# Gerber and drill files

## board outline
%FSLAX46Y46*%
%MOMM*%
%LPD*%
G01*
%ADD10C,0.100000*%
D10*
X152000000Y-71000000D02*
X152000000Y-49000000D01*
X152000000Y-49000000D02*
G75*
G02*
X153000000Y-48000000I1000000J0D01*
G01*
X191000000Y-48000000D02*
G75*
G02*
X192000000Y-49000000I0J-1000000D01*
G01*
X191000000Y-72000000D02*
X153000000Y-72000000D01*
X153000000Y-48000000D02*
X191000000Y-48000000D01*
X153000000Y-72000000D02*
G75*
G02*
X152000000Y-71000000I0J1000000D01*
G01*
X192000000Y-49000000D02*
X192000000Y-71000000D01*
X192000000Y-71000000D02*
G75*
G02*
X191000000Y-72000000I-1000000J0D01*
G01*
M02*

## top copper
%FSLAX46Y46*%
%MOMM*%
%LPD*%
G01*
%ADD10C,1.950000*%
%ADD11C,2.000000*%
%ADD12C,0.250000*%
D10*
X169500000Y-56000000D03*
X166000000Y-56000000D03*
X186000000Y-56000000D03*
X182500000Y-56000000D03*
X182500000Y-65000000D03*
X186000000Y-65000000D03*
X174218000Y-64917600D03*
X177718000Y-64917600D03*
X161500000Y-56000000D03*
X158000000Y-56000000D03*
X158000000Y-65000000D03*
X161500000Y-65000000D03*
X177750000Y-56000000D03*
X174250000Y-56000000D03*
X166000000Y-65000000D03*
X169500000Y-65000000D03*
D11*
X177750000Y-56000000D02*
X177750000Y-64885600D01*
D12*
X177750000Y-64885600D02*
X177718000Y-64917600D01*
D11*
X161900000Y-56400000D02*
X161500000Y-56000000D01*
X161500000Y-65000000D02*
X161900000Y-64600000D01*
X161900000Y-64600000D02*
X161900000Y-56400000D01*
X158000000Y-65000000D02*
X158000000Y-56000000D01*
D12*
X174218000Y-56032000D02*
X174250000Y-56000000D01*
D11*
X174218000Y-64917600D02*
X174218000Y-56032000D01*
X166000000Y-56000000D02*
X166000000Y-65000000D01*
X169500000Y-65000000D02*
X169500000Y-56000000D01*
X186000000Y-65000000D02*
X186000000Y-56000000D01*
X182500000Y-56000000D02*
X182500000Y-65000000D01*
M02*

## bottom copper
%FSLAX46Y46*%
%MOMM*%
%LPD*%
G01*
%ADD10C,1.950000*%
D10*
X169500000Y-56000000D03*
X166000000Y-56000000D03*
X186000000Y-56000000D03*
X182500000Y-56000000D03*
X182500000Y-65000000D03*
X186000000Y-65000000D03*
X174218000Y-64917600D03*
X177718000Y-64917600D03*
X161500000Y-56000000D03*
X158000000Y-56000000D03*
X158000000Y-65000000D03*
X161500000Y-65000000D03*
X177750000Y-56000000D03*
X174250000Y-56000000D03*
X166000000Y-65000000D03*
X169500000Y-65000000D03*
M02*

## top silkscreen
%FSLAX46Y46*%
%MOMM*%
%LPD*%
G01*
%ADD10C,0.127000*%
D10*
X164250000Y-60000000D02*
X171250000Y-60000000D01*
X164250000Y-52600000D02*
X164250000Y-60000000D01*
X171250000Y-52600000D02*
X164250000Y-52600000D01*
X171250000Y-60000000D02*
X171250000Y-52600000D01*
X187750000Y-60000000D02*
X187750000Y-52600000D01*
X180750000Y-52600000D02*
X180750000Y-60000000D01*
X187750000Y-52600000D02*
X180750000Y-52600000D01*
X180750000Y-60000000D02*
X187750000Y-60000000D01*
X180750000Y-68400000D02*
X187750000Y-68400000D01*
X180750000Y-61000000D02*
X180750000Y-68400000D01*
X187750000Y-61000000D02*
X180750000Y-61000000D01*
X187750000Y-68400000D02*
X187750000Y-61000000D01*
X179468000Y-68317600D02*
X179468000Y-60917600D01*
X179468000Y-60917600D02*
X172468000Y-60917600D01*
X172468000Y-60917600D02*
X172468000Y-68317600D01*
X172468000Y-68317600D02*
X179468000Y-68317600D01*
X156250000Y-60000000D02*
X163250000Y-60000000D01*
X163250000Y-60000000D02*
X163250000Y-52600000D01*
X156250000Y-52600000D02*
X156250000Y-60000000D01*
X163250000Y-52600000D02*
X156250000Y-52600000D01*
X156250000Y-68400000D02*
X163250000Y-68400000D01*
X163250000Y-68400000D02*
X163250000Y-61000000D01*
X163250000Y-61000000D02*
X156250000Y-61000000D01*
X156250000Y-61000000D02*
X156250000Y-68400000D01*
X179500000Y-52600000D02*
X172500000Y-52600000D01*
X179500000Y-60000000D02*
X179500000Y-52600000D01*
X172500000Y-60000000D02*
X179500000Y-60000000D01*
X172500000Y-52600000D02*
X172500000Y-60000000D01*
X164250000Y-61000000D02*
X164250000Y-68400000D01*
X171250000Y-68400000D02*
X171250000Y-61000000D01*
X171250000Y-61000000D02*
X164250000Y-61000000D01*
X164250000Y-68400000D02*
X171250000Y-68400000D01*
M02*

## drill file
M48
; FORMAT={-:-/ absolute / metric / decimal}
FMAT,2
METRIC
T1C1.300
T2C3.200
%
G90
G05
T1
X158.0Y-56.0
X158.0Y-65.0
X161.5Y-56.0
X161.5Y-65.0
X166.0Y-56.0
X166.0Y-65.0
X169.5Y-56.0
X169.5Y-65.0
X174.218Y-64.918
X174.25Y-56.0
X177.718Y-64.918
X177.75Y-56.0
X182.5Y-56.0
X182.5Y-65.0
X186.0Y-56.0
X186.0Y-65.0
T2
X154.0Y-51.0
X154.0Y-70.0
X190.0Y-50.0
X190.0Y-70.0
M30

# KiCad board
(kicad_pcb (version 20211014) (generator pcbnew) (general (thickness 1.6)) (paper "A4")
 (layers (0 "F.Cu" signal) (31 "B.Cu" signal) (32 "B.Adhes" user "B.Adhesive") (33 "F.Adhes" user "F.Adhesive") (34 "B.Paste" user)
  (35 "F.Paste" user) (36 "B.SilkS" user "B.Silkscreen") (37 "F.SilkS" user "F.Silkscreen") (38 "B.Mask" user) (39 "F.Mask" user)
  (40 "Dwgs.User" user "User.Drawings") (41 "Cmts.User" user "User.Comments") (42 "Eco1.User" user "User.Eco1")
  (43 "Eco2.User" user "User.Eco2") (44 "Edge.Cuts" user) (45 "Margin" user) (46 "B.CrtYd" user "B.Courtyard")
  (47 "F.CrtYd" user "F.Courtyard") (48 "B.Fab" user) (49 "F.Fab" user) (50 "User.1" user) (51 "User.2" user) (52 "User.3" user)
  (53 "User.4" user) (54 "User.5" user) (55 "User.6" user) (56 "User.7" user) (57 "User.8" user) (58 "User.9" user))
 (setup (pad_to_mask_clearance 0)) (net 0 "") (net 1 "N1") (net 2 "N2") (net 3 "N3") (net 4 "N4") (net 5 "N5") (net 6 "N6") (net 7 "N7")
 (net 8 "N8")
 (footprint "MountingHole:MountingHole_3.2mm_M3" (layer "F.Cu") (at 154 51)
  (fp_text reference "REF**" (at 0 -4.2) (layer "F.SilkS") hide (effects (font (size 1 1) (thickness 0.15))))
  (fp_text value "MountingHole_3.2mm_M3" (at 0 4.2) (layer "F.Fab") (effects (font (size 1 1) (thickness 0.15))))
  (pad "" np_thru_hole circle (at 0 0) (size 3.2 3.2) (drill 3.2) (layers *.Cu *.Mask)))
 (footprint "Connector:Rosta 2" (layer "F.Cu") (at 167.75 56 180)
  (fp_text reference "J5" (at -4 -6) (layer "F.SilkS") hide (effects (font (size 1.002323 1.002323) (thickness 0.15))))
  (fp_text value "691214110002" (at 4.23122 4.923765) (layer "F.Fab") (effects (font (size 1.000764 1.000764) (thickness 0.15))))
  (fp_line (start 3.5 -4) (end -3.5 -4) (layer "F.SilkS") (width 0.127))
  (fp_line (start 3.5 3.4) (end 3.5 -4) (layer "F.SilkS") (width 0.127))
  (fp_line (start -3.5 3.4) (end 3.5 3.4) (layer "F.SilkS") (width 0.127))
  (fp_line (start -3.5 -4) (end -3.5 3.4) (layer "F.SilkS") (width 0.127))
  (pad "1" thru_hole circle (at -1.75 0 180) (size 1.95 1.95) (drill 1.3) (layers *.Cu *.Mask) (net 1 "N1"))
  (pad "2" thru_hole circle (at 1.75 0 180) (size 1.95 1.95) (drill 1.3) (layers *.Cu *.Mask) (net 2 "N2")))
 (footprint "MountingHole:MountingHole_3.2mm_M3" (layer "F.Cu") (at 190 50)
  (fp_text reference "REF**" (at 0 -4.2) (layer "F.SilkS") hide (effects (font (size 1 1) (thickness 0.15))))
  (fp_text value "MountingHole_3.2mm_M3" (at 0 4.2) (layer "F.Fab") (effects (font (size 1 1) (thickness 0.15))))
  (pad "" np_thru_hole circle (at 0 0) (size 3.2 3.2) (drill 3.2) (layers *.Cu *.Mask)))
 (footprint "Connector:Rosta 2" (layer "F.Cu") (at 184.25 56 180)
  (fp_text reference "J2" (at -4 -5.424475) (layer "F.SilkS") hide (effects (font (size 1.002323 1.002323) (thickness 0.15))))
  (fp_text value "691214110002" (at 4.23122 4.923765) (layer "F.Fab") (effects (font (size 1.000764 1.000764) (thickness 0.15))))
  (fp_line (start -3.5 -4) (end -3.5 3.4) (layer "F.SilkS") (width 0.127))
  (fp_line (start 3.5 3.4) (end 3.5 -4) (layer "F.SilkS") (width 0.127))
  (fp_line (start -3.5 3.4) (end 3.5 3.4) (layer "F.SilkS") (width 0.127))
  (fp_line (start 3.5 -4) (end -3.5 -4) (layer "F.SilkS") (width 0.127))
  (pad "1" thru_hole circle (at -1.75 0 180) (size 1.95 1.95) (drill 1.3) (layers *.Cu *.Mask) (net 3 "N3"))
  (pad "2" thru_hole circle (at 1.75 0 180) (size 1.95 1.95) (drill 1.3) (layers *.Cu *.Mask) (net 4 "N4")))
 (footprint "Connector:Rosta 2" (layer "F.Cu") (at 184.25 65)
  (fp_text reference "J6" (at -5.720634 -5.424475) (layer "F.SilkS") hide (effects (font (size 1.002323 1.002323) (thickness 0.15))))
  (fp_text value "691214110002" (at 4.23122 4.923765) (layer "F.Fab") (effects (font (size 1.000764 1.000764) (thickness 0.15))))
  (fp_line (start -3.5 3.4) (end 3.5 3.4) (layer "F.SilkS") (width 0.127))
  (fp_line (start -3.5 -4) (end -3.5 3.4) (layer "F.SilkS") (width 0.127))
  (fp_line (start 3.5 -4) (end -3.5 -4) (layer "F.SilkS") (width 0.127))
  (fp_line (start 3.5 3.4) (end 3.5 -4) (layer "F.SilkS") (width 0.127))
  (pad "1" thru_hole circle (at -1.75 0) (size 1.95 1.95) (drill 1.3) (layers *.Cu *.Mask) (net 4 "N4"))
  (pad "2" thru_hole circle (at 1.75 0) (size 1.95 1.95) (drill 1.3) (layers *.Cu *.Mask) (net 3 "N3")))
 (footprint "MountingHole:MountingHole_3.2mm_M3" (layer "F.Cu") (at 154 70)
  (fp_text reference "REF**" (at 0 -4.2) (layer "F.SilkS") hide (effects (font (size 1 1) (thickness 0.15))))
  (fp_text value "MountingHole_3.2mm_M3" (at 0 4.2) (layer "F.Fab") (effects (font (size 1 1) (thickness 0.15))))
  (pad "" np_thru_hole circle (at 0 0) (size 3.2 3.2) (drill 3.2) (layers *.Cu *.Mask)))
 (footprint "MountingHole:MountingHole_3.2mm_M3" (layer "F.Cu") (at 190 70)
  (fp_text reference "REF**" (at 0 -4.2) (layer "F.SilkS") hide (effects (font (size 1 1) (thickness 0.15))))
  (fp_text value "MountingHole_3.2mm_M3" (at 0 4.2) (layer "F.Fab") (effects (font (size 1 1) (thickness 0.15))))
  (pad "" np_thru_hole circle (at 0 0) (size 3.2 3.2) (drill 3.2) (layers *.Cu *.Mask)))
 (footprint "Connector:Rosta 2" (layer "F.Cu") (at 175.968 64.9176)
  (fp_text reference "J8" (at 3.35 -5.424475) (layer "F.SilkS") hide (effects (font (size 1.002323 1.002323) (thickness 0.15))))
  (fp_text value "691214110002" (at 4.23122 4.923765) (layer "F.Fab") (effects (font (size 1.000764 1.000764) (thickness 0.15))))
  (fp_line (start 3.5 3.4) (end 3.5 -4) (layer "F.SilkS") (width 0.127))
  (fp_line (start 3.5 -4) (end -3.5 -4) (layer "F.SilkS") (width 0.127))
  (fp_line (start -3.5 -4) (end -3.5 3.4) (layer "F.SilkS") (width 0.127))
  (fp_line (start -3.5 3.4) (end 3.5 3.4) (layer "F.SilkS") (width 0.127))
  (pad "1" thru_hole circle (at -1.75 0) (size 1.95 1.95) (drill 1.3) (layers *.Cu *.Mask) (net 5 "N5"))
  (pad "2" thru_hole circle (at 1.75 0) (size 1.95 1.95) (drill 1.3) (layers *.Cu *.Mask) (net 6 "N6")))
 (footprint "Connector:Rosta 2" (layer "F.Cu") (at 159.75 56 180)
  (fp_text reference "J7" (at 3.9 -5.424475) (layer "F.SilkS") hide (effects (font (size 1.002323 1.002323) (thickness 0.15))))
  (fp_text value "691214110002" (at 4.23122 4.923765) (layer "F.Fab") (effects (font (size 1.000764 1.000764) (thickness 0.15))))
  (fp_line (start 3.5 -4) (end -3.5 -4) (layer "F.SilkS") (width 0.127))
  (fp_line (start -3.5 -4) (end -3.5 3.4) (layer "F.SilkS") (width 0.127))
  (fp_line (start 3.5 3.4) (end 3.5 -4) (layer "F.SilkS") (width 0.127))
  (fp_line (start -3.5 3.4) (end 3.5 3.4) (layer "F.SilkS") (width 0.127))
  (pad "1" thru_hole circle (at -1.75 0 180) (size 1.95 1.95) (drill 1.3) (layers *.Cu *.Mask) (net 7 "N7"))
  (pad "2" thru_hole circle (at 1.75 0 180) (size 1.95 1.95) (drill 1.3) (layers *.Cu *.Mask) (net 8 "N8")))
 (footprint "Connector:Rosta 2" (layer "F.Cu") (at 159.75 65)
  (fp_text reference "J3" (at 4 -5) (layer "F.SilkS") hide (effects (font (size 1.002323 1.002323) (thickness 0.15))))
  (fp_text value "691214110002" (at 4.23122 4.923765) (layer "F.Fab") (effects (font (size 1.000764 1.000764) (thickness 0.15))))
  (fp_line (start -3.5 3.4) (end 3.5 3.4) (layer "F.SilkS") (width 0.127))
  (fp_line (start 3.5 3.4) (end 3.5 -4) (layer "F.SilkS") (width 0.127))
  (fp_line (start 3.5 -4) (end -3.5 -4) (layer "F.SilkS") (width 0.127))
  (fp_line (start -3.5 -4) (end -3.5 3.4) (layer "F.SilkS") (width 0.127))
  (pad "1" thru_hole circle (at -1.75 0) (size 1.95 1.95) (drill 1.3) (layers *.Cu *.Mask) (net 8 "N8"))
  (pad "2" thru_hole circle (at 1.75 0) (size 1.95 1.95) (drill 1.3) (layers *.Cu *.Mask) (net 7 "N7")))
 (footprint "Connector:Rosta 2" (layer "F.Cu") (at 176 56 180)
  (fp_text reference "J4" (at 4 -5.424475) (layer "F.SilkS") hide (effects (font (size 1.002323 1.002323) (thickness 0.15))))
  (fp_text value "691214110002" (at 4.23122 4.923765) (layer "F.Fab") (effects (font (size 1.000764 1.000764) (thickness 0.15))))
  (fp_line (start -3.5 3.4) (end 3.5 3.4) (layer "F.SilkS") (width 0.127))
  (fp_line (start -3.5 -4) (end -3.5 3.4) (layer "F.SilkS") (width 0.127))
  (fp_line (start 3.5 -4) (end -3.5 -4) (layer "F.SilkS") (width 0.127))
  (fp_line (start 3.5 3.4) (end 3.5 -4) (layer "F.SilkS") (width 0.127))
  (pad "1" thru_hole circle (at -1.75 0 180) (size 1.95 1.95) (drill 1.3) (layers *.Cu *.Mask) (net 6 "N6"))
  (pad "2" thru_hole circle (at 1.75 0 180) (size 1.95 1.95) (drill 1.3) (layers *.Cu *.Mask) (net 5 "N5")))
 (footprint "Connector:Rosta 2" (layer "F.Cu") (at 167.75 65)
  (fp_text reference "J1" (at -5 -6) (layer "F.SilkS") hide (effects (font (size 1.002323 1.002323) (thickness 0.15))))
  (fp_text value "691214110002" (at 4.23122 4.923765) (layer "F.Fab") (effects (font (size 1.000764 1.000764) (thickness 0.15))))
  (fp_line (start -3.5 -4) (end -3.5 3.4) (layer "F.SilkS") (width 0.127))
  (fp_line (start 3.5 3.4) (end 3.5 -4) (layer "F.SilkS") (width 0.127))
  (fp_line (start 3.5 -4) (end -3.5 -4) (layer "F.SilkS") (width 0.127))
  (fp_line (start -3.5 3.4) (end 3.5 3.4) (layer "F.SilkS") (width 0.127))
  (pad "1" thru_hole circle (at -1.75 0) (size 1.95 1.95) (drill 1.3) (layers *.Cu *.Mask) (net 2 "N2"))
  (pad "2" thru_hole circle (at 1.75 0) (size 1.95 1.95) (drill 1.3) (layers *.Cu *.Mask) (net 1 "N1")))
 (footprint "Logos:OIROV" (layer "B.Cu") (at 172 60 180)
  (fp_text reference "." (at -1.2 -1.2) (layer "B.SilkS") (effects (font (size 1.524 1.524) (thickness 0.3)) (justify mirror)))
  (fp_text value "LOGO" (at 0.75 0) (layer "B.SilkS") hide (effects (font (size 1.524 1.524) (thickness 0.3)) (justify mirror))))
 (gr_line (start 152 71) (end 152 49) (layer "Edge.Cuts") (width 0.1))
 (gr_arc (start 152 49) (mid 152.292893 48.292893) (end 153 48) (layer "Edge.Cuts") (width 0.1))
 (gr_arc (start 191 48) (mid 191.707107 48.292893) (end 192 49) (layer "Edge.Cuts") (width 0.1))
 (gr_line (start 191 72) (end 153 72) (layer "Edge.Cuts") (width 0.1))
 (gr_line (start 153 48) (end 191 48) (layer "Edge.Cuts") (width 0.1))
 (gr_arc (start 153 72) (mid 152.292893 71.707107) (end 152 71) (layer "Edge.Cuts") (width 0.1))
 (gr_line (start 192 49) (end 192 71) (layer "Edge.Cuts") (width 0.1))
 (gr_arc (start 192 71) (mid 191.707107 71.707107) (end 191 72) (layer "Edge.Cuts") (width 0.1))
 (segment (start 177.75 56) (end 177.75 64.8856) (width 2) (layer "F.Cu") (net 6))
 (segment (start 177.75 64.8856) (end 177.718 64.9176) (width 0.25) (layer "F.Cu") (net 6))
 (segment (start 161.9 56.4) (end 161.5 56) (width 2) (layer "F.Cu") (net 7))
 (segment (start 161.5 65) (end 161.9 64.6) (width 2) (layer "F.Cu") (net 7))
 (segment (start 161.9 64.6) (end 161.9 56.4) (width 2) (layer "F.Cu") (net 7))
 (segment (start 158 65) (end 158 56) (width 2) (layer "F.Cu") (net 8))
 (segment (start 174.218 56.032) (end 174.25 56) (width 0.25) (layer "F.Cu") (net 5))
 (segment (start 174.218 64.9176) (end 174.218 56.032) (width 2) (layer "F.Cu") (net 5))
 (segment (start 166 56) (end 166 65) (width 2) (layer "F.Cu") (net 2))
 (segment (start 169.5 65) (end 169.5 56) (width 2) (layer "F.Cu") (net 1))
 (segment (start 186 65) (end 186 56) (width 2) (layer "F.Cu") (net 3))
 (segment (start 182.5 56) (end 182.5 65) (width 2) (layer "F.Cu") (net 4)))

